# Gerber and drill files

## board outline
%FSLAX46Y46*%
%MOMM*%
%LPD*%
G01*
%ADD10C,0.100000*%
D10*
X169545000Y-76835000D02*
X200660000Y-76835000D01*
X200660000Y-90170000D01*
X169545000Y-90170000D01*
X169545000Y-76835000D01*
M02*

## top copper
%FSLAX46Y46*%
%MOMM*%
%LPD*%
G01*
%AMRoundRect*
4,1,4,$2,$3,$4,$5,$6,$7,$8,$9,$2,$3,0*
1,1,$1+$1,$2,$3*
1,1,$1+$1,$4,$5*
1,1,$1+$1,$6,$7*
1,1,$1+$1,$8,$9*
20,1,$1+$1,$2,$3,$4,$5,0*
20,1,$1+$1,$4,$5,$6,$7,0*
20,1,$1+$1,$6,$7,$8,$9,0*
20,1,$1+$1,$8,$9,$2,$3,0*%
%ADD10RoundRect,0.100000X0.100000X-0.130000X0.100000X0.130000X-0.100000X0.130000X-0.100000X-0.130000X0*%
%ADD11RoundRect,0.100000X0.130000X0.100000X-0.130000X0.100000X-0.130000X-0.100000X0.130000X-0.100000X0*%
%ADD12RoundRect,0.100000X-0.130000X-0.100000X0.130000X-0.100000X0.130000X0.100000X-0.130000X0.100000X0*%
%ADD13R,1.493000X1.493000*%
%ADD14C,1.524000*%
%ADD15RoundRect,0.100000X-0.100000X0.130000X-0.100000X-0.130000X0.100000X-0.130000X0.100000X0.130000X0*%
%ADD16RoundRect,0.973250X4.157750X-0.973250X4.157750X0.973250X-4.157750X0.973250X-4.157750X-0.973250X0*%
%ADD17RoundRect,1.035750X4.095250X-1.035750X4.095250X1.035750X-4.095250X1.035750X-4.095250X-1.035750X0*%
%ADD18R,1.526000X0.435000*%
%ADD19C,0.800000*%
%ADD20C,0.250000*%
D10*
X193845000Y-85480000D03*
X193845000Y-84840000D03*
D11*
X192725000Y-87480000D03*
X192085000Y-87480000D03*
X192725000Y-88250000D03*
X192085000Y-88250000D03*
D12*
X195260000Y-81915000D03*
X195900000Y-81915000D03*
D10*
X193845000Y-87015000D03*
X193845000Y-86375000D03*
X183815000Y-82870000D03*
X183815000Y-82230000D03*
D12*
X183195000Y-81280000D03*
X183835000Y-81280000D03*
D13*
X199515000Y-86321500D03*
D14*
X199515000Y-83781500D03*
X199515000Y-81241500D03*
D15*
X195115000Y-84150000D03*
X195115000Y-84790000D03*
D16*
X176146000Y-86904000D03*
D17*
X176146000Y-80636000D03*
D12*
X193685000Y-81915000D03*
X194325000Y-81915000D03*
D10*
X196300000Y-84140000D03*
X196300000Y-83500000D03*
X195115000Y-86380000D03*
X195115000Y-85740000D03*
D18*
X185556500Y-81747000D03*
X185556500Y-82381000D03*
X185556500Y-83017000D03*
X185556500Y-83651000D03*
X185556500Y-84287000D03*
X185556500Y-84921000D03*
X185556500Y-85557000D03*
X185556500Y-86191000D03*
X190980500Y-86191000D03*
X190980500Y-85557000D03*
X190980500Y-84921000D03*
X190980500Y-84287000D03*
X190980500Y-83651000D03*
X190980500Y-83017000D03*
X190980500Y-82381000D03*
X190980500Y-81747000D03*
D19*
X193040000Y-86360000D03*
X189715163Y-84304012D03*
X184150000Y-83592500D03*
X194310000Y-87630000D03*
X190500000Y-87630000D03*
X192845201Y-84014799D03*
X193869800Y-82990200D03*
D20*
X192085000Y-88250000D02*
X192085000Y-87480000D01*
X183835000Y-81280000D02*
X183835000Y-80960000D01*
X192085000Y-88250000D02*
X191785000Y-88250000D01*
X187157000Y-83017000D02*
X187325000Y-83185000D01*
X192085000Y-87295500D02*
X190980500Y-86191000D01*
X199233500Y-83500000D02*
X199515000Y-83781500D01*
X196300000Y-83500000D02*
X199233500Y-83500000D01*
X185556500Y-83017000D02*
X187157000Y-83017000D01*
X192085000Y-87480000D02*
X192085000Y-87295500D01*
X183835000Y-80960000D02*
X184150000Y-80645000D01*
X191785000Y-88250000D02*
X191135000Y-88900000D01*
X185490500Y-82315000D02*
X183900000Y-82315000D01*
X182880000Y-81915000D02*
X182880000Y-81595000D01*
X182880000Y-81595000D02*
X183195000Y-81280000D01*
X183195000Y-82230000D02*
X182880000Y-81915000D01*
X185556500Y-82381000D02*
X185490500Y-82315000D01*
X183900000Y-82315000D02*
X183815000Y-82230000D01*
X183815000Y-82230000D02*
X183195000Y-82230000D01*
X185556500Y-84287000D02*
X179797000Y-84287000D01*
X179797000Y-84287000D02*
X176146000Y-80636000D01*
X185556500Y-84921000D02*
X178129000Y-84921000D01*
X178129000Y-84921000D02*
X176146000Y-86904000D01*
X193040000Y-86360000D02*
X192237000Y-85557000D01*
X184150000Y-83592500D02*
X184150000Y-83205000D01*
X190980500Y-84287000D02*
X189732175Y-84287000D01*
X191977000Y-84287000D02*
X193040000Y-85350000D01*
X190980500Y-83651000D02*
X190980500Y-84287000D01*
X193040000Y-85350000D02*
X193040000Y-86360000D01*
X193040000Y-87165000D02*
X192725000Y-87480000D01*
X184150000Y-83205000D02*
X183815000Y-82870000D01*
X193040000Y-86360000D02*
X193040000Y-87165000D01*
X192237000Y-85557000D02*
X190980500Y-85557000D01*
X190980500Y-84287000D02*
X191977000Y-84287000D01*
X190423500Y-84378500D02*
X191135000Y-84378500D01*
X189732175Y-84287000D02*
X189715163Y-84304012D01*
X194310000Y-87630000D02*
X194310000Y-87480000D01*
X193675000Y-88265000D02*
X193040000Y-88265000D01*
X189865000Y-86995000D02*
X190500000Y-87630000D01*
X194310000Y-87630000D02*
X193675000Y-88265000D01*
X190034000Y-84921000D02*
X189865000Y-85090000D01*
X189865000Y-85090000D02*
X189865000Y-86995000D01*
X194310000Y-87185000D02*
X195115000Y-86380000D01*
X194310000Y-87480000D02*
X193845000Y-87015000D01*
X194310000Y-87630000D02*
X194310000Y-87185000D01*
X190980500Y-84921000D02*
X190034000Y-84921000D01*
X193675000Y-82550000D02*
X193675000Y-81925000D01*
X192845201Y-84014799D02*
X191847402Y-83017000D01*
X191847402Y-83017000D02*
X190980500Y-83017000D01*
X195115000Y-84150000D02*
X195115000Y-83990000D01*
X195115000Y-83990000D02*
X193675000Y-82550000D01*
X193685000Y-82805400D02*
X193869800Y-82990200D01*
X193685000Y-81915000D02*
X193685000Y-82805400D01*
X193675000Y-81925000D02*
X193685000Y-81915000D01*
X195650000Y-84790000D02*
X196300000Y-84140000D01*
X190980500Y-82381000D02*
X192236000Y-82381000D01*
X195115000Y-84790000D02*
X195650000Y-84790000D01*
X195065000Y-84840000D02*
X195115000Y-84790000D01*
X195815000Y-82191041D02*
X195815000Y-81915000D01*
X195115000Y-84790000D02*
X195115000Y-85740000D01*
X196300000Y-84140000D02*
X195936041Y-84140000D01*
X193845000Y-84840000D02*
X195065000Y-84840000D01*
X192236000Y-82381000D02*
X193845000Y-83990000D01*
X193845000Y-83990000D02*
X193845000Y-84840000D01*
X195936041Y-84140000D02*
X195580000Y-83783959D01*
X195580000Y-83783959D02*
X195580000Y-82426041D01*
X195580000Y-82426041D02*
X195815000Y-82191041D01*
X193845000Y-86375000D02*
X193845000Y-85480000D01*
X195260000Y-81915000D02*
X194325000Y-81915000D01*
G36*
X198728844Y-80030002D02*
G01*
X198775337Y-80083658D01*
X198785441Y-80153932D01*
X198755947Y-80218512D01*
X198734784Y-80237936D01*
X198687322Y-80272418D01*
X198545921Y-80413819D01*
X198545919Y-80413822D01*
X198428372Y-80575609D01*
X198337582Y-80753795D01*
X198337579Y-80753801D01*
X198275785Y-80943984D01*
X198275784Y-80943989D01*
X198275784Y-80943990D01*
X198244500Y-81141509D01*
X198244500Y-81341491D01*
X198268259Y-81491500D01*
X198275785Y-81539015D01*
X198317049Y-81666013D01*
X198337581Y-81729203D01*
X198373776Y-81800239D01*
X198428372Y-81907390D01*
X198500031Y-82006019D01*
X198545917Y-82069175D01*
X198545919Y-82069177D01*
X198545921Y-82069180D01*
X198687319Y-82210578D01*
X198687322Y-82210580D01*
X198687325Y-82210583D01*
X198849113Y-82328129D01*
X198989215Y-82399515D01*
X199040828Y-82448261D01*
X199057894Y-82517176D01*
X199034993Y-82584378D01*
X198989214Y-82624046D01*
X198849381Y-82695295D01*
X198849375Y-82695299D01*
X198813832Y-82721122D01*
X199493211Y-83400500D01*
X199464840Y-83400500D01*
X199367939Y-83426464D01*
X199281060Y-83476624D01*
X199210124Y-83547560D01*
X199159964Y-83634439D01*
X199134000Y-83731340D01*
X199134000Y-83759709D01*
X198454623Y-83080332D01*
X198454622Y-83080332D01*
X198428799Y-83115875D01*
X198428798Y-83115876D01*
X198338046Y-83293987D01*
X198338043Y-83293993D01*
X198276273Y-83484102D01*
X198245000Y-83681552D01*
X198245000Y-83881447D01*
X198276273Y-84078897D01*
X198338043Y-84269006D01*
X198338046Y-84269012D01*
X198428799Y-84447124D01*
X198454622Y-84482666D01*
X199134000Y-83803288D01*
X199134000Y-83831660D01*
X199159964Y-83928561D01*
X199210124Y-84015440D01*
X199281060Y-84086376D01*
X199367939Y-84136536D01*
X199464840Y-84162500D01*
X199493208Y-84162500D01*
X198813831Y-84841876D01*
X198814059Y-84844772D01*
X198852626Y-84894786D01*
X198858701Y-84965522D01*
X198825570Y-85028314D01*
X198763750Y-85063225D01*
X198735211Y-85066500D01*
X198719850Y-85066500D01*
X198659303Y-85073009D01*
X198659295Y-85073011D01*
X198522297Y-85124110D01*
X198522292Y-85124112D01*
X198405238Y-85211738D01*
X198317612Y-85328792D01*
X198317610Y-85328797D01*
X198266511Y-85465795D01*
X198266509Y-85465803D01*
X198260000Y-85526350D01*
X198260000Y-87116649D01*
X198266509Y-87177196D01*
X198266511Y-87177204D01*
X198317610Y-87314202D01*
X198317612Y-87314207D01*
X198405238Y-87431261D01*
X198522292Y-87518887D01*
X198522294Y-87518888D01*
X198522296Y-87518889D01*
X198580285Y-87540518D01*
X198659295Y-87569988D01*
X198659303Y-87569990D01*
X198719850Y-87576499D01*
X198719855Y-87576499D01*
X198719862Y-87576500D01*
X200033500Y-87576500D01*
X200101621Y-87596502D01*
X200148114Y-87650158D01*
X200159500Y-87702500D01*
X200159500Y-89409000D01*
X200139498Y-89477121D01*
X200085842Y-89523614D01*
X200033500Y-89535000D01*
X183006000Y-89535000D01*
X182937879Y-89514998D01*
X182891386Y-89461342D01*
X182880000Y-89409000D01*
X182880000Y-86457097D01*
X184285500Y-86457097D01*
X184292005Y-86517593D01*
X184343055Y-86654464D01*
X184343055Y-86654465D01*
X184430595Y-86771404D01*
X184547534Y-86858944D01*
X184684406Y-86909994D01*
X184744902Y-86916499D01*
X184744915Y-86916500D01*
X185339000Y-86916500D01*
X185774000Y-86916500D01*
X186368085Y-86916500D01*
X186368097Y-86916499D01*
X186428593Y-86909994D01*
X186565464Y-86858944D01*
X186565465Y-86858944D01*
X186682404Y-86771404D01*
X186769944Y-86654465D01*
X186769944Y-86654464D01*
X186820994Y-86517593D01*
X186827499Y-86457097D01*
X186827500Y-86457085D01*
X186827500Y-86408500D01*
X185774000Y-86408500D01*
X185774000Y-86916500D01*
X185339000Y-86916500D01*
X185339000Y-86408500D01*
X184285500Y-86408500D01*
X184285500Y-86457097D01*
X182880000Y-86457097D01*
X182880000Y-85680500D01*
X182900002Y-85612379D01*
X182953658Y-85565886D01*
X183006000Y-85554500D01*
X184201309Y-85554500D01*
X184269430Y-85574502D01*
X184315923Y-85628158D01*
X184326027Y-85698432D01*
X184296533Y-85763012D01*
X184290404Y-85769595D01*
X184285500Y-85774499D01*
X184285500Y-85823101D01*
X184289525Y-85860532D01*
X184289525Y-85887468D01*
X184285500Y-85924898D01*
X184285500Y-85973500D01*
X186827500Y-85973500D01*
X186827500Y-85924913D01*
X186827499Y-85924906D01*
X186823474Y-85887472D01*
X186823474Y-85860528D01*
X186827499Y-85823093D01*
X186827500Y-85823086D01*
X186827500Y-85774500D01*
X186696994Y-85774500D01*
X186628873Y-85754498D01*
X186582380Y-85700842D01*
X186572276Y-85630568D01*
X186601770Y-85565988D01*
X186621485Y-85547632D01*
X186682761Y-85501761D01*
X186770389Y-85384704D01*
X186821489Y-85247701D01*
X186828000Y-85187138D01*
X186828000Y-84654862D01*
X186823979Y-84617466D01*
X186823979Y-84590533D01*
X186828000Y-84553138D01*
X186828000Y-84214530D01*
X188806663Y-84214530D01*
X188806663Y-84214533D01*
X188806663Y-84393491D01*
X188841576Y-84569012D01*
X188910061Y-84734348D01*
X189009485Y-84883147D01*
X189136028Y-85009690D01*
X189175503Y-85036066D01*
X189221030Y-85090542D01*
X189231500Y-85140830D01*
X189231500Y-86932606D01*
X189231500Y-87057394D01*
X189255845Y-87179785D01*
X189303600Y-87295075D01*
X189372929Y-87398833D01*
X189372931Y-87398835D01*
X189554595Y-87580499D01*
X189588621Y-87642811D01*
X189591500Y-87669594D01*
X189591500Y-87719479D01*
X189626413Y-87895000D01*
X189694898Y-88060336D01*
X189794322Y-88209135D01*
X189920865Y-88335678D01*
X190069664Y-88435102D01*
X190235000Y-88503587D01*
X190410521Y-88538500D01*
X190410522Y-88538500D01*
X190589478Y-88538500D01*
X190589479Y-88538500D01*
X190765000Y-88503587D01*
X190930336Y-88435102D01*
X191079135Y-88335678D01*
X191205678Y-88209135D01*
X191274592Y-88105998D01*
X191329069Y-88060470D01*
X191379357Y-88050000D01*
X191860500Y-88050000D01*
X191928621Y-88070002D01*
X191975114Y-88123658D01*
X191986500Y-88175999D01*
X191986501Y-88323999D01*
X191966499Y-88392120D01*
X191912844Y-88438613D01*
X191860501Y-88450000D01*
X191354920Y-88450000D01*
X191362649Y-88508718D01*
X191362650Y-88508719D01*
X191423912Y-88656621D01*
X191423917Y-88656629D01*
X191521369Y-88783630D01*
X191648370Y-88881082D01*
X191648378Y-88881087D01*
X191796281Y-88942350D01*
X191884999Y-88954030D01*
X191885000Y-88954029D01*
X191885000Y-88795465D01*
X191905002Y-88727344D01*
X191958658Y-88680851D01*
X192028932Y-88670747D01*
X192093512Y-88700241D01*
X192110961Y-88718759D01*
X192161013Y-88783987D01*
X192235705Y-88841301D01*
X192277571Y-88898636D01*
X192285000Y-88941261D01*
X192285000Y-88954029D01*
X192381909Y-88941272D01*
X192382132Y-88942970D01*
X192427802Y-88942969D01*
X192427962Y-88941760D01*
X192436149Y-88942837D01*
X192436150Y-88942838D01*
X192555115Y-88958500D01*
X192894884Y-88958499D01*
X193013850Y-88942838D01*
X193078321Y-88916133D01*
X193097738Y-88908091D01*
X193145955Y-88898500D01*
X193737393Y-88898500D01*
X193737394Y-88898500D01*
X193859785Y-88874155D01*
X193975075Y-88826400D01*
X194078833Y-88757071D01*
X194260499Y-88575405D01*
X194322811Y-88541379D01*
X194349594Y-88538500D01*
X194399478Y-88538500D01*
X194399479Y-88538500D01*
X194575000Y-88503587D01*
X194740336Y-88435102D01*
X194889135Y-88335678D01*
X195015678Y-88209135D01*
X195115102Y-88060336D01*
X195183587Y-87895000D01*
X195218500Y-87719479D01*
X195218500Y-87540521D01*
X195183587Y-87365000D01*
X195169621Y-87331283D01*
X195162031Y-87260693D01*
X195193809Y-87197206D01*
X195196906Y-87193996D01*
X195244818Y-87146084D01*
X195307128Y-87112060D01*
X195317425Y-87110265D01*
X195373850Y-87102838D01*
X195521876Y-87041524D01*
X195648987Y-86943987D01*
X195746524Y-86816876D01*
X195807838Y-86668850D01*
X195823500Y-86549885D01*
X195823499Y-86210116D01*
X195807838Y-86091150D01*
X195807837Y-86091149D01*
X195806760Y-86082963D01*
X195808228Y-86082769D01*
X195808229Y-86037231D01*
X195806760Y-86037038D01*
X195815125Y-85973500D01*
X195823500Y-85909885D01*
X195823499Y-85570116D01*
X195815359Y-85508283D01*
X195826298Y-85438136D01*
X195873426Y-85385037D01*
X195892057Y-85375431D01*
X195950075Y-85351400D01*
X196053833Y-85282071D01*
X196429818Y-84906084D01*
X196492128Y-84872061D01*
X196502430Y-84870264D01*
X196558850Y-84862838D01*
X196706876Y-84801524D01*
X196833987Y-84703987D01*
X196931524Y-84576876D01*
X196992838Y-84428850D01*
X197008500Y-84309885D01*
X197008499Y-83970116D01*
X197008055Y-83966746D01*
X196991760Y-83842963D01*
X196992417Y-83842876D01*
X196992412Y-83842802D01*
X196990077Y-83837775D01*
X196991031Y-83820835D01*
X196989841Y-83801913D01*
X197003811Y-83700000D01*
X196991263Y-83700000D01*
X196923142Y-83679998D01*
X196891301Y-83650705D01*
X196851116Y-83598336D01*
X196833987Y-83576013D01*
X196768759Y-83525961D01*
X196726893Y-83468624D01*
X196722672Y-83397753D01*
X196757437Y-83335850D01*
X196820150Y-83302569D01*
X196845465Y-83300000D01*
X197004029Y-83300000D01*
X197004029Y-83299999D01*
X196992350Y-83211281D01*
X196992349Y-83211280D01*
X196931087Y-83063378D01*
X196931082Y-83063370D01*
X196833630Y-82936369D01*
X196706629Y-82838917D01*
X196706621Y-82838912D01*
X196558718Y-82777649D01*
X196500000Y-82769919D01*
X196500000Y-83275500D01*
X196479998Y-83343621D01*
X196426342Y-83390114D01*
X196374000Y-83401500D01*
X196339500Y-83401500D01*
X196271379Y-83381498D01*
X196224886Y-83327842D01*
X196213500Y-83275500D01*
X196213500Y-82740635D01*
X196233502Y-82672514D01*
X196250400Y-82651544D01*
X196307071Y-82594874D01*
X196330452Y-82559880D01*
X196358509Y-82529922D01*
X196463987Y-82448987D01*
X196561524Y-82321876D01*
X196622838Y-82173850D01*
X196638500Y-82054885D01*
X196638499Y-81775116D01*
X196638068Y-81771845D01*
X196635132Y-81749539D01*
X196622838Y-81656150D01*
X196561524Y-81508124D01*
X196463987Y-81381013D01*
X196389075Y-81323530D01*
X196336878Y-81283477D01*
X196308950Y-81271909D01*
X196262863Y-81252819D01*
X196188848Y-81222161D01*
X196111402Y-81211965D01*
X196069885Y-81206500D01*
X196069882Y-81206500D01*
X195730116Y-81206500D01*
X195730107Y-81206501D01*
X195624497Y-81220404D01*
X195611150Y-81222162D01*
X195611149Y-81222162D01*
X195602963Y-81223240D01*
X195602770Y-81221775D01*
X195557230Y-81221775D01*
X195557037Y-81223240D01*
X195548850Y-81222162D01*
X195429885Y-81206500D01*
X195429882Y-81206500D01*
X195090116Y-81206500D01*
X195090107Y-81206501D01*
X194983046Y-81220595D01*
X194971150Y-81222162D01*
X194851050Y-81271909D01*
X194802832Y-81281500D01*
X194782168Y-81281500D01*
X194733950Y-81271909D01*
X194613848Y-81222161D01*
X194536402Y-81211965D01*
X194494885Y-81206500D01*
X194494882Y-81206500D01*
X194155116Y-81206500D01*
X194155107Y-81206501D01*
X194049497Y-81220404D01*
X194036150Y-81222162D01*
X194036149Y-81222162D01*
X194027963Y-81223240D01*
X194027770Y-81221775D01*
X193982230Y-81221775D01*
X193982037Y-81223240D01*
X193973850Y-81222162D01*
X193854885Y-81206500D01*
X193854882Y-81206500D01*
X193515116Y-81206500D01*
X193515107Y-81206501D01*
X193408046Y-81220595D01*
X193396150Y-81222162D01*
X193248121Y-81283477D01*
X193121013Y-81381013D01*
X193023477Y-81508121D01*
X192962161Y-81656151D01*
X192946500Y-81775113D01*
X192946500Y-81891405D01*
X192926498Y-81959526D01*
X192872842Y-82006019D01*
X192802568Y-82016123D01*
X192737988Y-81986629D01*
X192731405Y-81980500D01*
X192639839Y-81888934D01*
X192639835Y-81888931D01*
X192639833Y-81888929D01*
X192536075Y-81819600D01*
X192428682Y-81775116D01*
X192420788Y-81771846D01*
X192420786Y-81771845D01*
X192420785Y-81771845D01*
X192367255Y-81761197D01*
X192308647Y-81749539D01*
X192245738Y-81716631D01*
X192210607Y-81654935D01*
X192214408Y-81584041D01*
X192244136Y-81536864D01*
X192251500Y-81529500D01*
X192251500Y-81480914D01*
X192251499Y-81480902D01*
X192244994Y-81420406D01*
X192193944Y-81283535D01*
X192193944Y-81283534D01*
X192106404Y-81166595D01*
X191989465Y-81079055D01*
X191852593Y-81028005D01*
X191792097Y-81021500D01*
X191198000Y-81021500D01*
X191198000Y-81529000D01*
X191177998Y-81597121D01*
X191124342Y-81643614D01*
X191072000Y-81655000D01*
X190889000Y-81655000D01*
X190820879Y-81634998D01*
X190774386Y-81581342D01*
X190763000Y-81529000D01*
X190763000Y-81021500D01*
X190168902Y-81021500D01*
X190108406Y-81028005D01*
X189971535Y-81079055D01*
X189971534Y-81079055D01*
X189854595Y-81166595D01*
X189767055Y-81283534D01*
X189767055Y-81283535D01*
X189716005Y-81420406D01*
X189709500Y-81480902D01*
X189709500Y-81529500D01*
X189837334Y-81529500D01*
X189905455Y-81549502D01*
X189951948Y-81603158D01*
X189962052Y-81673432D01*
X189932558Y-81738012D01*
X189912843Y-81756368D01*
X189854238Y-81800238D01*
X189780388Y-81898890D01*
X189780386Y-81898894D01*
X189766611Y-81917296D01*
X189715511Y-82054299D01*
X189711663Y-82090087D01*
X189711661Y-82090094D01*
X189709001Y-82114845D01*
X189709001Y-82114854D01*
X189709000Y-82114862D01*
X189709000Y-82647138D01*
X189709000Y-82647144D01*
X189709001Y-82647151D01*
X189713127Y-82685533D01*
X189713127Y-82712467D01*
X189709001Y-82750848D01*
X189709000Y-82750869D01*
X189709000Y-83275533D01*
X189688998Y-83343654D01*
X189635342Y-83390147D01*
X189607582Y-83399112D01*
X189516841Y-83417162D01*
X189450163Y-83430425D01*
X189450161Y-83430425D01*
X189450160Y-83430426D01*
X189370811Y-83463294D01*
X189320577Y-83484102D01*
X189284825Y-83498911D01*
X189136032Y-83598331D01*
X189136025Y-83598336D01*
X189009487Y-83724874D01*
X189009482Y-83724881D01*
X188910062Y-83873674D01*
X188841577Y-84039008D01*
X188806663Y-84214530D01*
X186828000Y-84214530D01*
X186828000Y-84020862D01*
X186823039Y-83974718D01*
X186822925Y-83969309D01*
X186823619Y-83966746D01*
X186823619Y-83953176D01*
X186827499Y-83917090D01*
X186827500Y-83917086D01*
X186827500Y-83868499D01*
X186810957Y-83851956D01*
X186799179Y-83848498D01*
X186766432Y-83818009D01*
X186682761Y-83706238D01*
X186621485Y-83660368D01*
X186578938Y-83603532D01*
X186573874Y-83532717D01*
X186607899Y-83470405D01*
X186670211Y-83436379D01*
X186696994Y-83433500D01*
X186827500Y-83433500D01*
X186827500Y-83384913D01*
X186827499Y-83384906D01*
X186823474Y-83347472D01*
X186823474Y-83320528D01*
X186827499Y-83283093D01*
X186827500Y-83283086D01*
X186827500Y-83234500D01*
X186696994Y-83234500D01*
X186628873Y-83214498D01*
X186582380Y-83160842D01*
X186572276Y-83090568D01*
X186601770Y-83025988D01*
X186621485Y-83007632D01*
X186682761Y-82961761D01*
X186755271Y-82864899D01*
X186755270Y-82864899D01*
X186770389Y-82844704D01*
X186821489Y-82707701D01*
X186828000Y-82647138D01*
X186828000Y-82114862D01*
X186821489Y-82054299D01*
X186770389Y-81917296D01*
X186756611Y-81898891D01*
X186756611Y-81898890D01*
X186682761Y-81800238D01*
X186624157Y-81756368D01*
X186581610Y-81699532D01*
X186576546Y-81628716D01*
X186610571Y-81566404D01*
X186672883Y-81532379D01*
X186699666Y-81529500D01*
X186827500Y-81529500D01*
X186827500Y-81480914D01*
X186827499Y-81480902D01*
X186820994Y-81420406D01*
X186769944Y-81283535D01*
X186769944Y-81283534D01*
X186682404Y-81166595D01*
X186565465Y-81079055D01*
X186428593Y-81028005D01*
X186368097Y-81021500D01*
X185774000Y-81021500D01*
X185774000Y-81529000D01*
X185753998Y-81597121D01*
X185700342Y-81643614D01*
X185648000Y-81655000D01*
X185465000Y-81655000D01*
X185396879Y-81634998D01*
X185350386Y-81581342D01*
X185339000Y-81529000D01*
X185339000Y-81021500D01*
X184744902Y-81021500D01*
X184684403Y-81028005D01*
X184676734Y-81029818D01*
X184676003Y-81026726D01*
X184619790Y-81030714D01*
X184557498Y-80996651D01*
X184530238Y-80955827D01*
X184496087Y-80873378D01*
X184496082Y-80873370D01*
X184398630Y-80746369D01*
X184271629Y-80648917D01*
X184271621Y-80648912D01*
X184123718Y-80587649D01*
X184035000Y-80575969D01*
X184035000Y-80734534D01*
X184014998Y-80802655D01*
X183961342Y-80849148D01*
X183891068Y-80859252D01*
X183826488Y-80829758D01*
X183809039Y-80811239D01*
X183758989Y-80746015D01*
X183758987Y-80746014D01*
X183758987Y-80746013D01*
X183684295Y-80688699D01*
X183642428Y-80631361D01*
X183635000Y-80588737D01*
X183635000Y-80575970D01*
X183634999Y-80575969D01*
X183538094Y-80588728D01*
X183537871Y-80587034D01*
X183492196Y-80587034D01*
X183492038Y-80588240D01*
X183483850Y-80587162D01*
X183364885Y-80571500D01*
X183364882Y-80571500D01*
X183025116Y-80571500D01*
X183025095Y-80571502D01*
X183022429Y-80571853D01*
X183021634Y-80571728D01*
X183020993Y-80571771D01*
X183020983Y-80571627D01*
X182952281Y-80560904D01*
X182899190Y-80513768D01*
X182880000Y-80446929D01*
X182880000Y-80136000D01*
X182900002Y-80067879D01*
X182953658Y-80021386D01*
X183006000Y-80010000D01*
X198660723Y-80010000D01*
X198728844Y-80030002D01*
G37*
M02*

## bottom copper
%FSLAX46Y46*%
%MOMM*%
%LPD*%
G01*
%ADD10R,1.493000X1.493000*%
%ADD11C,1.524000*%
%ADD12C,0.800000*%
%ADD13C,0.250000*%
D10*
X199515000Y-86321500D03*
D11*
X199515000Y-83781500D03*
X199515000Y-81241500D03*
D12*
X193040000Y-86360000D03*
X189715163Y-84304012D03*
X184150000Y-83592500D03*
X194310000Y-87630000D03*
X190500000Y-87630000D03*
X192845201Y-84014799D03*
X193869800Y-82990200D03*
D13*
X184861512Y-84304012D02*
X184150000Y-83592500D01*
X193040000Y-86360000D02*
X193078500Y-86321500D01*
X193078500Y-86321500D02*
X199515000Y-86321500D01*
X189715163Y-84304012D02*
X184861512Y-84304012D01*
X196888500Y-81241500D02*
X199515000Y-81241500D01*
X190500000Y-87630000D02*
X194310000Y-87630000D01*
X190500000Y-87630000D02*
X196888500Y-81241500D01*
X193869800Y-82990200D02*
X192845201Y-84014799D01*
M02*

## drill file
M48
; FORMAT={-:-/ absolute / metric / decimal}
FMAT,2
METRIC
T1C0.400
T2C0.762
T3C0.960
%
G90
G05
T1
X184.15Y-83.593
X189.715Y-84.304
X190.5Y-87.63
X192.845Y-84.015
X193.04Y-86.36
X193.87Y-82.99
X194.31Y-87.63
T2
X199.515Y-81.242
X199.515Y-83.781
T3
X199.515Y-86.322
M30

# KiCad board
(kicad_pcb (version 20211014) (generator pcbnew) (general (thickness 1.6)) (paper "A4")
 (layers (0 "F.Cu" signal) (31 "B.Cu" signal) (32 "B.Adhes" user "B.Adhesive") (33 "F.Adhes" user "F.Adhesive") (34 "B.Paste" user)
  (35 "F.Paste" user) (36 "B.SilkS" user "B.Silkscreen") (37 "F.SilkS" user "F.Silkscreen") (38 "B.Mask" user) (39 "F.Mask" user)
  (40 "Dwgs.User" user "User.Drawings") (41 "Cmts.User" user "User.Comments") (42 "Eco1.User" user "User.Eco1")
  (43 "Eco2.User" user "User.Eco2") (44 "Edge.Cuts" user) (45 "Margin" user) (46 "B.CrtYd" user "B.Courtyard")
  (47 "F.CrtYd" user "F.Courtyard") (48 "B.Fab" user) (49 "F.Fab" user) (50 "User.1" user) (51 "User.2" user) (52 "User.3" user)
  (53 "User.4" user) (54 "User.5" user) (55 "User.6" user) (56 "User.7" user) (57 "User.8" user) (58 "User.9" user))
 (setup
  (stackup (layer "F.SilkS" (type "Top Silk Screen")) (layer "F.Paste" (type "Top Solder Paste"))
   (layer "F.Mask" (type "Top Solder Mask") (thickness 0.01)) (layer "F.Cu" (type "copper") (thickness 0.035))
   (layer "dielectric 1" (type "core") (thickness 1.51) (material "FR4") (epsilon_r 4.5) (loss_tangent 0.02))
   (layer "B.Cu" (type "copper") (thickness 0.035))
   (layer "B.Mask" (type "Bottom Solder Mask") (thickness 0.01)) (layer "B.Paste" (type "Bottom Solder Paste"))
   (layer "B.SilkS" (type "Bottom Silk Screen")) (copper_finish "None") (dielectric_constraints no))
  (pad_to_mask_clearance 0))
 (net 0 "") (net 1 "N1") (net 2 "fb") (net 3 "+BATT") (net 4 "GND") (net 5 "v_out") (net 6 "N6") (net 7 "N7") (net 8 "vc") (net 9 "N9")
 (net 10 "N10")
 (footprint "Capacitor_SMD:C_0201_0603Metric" (layer "F.Cu") (at 193.845 85.16 90)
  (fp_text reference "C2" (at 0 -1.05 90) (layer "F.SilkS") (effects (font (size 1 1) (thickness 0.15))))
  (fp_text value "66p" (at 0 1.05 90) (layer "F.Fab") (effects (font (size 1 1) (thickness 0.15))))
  (pad "" smd roundrect (at 0.345 0 90) (size 0.318 0.36) (layers "F.Paste") (roundrect_rratio 0.25))
  (pad "" smd roundrect (at -0.345 0 90) (size 0.318 0.36) (layers "F.Paste") (roundrect_rratio 0.25))
  (pad "1" smd roundrect (at -0.32 0 90) (size 0.46 0.4) (layers "F.Cu" "F.Mask") (roundrect_rratio 0.25) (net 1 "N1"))
  (pad "2" smd roundrect (at 0.32 0 90) (size 0.46 0.4) (layers "F.Cu" "F.Mask") (roundrect_rratio 0.25) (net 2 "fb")))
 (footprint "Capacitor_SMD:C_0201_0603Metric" (layer "F.Cu") (at 192.405 87.48 180)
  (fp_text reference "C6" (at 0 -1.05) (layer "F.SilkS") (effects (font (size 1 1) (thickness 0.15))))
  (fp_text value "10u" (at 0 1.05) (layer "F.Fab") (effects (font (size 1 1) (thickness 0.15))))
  (pad "" smd roundrect (at -0.345 0 180) (size 0.318 0.36) (layers "F.Paste") (roundrect_rratio 0.25))
  (pad "" smd roundrect (at 0.345 0 180) (size 0.318 0.36) (layers "F.Paste") (roundrect_rratio 0.25))
  (pad "1" smd roundrect (at -0.32 0 180) (size 0.46 0.4) (layers "F.Cu" "F.Mask") (roundrect_rratio 0.25) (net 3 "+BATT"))
  (pad "2" smd roundrect (at 0.32 0 180) (size 0.46 0.4) (layers "F.Cu" "F.Mask") (roundrect_rratio 0.25) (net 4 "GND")))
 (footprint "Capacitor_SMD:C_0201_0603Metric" (layer "F.Cu") (at 192.405 88.25 180)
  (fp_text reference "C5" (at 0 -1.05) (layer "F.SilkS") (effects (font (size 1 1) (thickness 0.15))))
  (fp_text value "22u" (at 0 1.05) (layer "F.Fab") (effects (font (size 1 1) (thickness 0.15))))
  (pad "" smd roundrect (at 0.345 0 180) (size 0.318 0.36) (layers "F.Paste") (roundrect_rratio 0.25))
  (pad "" smd roundrect (at -0.345 0 180) (size 0.318 0.36) (layers "F.Paste") (roundrect_rratio 0.25))
  (pad "1" smd roundrect (at -0.32 0 180) (size 0.46 0.4) (layers "F.Cu" "F.Mask") (roundrect_rratio 0.25) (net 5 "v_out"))
  (pad "2" smd roundrect (at 0.32 0 180) (size 0.46 0.4) (layers "F.Cu" "F.Mask") (roundrect_rratio 0.25) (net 4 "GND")))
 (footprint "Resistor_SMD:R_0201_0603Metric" (layer "F.Cu") (at 195.58 81.915)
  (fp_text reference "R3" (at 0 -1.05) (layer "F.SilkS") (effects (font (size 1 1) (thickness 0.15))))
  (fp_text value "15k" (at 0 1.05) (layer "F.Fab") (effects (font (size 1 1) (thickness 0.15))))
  (pad "" smd roundrect (at -0.345 0) (size 0.318 0.36) (layers "F.Paste") (roundrect_rratio 0.25))
  (pad "" smd roundrect (at 0.345 0) (size 0.318 0.36) (layers "F.Paste") (roundrect_rratio 0.25))
  (pad "1" smd roundrect (at -0.32 0) (size 0.46 0.4) (layers "F.Cu" "F.Mask") (roundrect_rratio 0.25) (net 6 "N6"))
  (pad "2" smd roundrect (at 0.32 0) (size 0.46 0.4) (layers "F.Cu" "F.Mask") (roundrect_rratio 0.25) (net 2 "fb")))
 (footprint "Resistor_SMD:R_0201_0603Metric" (layer "F.Cu") (at 193.845 86.695 90)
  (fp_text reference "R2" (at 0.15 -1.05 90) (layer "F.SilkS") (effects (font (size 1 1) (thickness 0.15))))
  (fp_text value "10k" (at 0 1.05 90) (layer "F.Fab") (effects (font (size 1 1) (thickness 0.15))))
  (pad "" smd roundrect (at -0.345 0 90) (size 0.318 0.36) (layers "F.Paste") (roundrect_rratio 0.25))
  (pad "" smd roundrect (at 0.345 0 90) (size 0.318 0.36) (layers "F.Paste") (roundrect_rratio 0.25))
  (pad "1" smd roundrect (at -0.32 0 90) (size 0.46 0.4) (layers "F.Cu" "F.Mask") (roundrect_rratio 0.25) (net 5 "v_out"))
  (pad "2" smd roundrect (at 0.32 0 90) (size 0.46 0.4) (layers "F.Cu" "F.Mask") (roundrect_rratio 0.25) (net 1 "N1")))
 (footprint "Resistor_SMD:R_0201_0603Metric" (layer "F.Cu") (at 183.815 82.55 90)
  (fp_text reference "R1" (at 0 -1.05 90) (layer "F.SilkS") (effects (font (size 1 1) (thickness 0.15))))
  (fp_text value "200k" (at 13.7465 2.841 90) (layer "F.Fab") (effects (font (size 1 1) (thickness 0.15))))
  (pad "" smd roundrect (at -0.345 0 90) (size 0.318 0.36) (layers "F.Paste") (roundrect_rratio 0.25))
  (pad "" smd roundrect (at 0.345 0 90) (size 0.318 0.36) (layers "F.Paste") (roundrect_rratio 0.25))
  (pad "1" smd roundrect (at -0.32 0 90) (size 0.46 0.4) (layers "F.Cu" "F.Mask") (roundrect_rratio 0.25) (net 3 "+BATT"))
  (pad "2" smd roundrect (at 0.32 0 90) (size 0.46 0.4) (layers "F.Cu" "F.Mask") (roundrect_rratio 0.25) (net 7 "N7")))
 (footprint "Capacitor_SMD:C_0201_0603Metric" (layer "F.Cu") (at 183.515 81.28)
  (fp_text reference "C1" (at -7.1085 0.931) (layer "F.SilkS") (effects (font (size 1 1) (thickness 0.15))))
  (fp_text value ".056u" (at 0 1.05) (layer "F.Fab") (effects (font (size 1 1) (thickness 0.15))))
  (pad "" smd roundrect (at 0.345 0) (size 0.318 0.36) (layers "F.Paste") (roundrect_rratio 0.25))
  (pad "" smd roundrect (at -0.345 0) (size 0.318 0.36) (layers "F.Paste") (roundrect_rratio 0.25))
  (pad "1" smd roundrect (at -0.32 0) (size 0.46 0.4) (layers "F.Cu" "F.Mask") (roundrect_rratio 0.25) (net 7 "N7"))
  (pad "2" smd roundrect (at 0.32 0) (size 0.46 0.4) (layers "F.Cu" "F.Mask") (roundrect_rratio 0.25) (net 4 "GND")))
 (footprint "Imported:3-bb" (layer "F.Cu") (at 199.515 86.3215 90)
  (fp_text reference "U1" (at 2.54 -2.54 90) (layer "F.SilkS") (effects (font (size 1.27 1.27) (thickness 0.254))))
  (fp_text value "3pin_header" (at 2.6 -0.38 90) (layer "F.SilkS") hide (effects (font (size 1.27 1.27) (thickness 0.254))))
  (pad "1" thru_hole rect (at 0 0 90) (size 1.493 1.493) (drill 0.96) (layers *.Cu *.Mask) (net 3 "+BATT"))
  (pad "2" thru_hole circle (at 2.54 0 90) (size 1.524 1.524) (drill 0.762) (layers *.Cu *.Mask) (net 4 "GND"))
  (pad "3" thru_hole circle (at 5.08 0 90) (size 1.524 1.524) (drill 0.762) (layers *.Cu *.Mask) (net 5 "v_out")))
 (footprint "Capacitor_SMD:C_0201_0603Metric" (layer "F.Cu") (at 195.115 84.47 -90)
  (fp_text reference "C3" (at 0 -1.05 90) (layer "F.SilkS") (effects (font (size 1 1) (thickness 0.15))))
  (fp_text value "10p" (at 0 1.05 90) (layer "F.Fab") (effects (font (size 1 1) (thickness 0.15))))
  (pad "" smd roundrect (at -0.345 0 270) (size 0.318 0.36) (layers "F.Paste") (roundrect_rratio 0.25))
  (pad "" smd roundrect (at 0.345 0 270) (size 0.318 0.36) (layers "F.Paste") (roundrect_rratio 0.25))
  (pad "1" smd roundrect (at -0.32 0 270) (size 0.46 0.4) (layers "F.Cu" "F.Mask") (roundrect_rratio 0.25) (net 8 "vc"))
  (pad "2" smd roundrect (at 0.32 0 270) (size 0.46 0.4) (layers "F.Cu" "F.Mask") (roundrect_rratio 0.25) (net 2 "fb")))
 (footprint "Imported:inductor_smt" (layer "F.Cu") (at 183.515 91.2075 90)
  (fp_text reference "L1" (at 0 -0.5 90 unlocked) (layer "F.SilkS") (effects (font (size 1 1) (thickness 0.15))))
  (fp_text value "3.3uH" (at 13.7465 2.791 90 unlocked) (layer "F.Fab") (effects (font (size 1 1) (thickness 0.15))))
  (pad "1" smd roundrect (at 4.3035 -7.369 90) (size 3.893 10.262) (layers "F.Cu" "F.Paste" "F.Mask") (roundrect_rratio 0.25) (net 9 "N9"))
  (pad "2" smd roundrect (at 10.5715 -7.369 90) (size 4.143 10.262) (layers "F.Cu" "F.Paste" "F.Mask") (roundrect_rratio 0.25)
   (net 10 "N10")))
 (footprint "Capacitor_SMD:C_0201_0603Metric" (layer "F.Cu") (at 194.005 81.915)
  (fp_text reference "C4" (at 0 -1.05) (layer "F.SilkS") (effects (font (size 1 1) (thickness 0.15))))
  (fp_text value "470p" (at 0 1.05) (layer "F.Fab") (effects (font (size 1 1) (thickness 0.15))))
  (pad "" smd roundrect (at -0.345 0) (size 0.318 0.36) (layers "F.Paste") (roundrect_rratio 0.25))
  (pad "" smd roundrect (at 0.345 0) (size 0.318 0.36) (layers "F.Paste") (roundrect_rratio 0.25))
  (pad "1" smd roundrect (at -0.32 0) (size 0.46 0.4) (layers "F.Cu" "F.Mask") (roundrect_rratio 0.25) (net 8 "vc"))
  (pad "2" smd roundrect (at 0.32 0) (size 0.46 0.4) (layers "F.Cu" "F.Mask") (roundrect_rratio 0.25) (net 6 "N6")))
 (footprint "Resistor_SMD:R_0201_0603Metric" (layer "F.Cu") (at 196.3 83.82 90)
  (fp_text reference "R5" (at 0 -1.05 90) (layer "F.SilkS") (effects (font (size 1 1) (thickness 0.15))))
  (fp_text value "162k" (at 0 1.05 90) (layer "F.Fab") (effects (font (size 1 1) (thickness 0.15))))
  (pad "" smd roundrect (at 0.345 0 90) (size 0.318 0.36) (layers "F.Paste") (roundrect_rratio 0.25))
  (pad "" smd roundrect (at -0.345 0 90) (size 0.318 0.36) (layers "F.Paste") (roundrect_rratio 0.25))
  (pad "1" smd roundrect (at -0.32 0 90) (size 0.46 0.4) (layers "F.Cu" "F.Mask") (roundrect_rratio 0.25) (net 2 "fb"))
  (pad "2" smd roundrect (at 0.32 0 90) (size 0.46 0.4) (layers "F.Cu" "F.Mask") (roundrect_rratio 0.25) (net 4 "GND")))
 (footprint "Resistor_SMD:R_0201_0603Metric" (layer "F.Cu") (at 195.115 86.06 90)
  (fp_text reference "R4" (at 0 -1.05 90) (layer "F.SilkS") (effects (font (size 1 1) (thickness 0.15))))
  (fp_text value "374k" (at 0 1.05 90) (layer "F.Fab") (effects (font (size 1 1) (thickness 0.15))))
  (pad "" smd roundrect (at 0.345 0 90) (size 0.318 0.36) (layers "F.Paste") (roundrect_rratio 0.25))
  (pad "" smd roundrect (at -0.345 0 90) (size 0.318 0.36) (layers "F.Paste") (roundrect_rratio 0.25))
  (pad "1" smd roundrect (at -0.32 0 90) (size 0.46 0.4) (layers "F.Cu" "F.Mask") (roundrect_rratio 0.25) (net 5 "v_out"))
  (pad "2" smd roundrect (at 0.32 0 90) (size 0.46 0.4) (layers "F.Cu" "F.Mask") (roundrect_rratio 0.25) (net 2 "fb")))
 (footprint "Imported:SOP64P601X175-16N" (layer "F.Cu") (at 188.2685 83.969)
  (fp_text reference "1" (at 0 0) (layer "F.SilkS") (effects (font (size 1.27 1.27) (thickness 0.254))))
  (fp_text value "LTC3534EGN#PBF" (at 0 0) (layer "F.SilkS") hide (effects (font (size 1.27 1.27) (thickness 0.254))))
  (pad "1" smd rect (at -2.712 -2.222 90) (size 0.435 1.526) (layers "F.Cu" "F.Paste" "F.Mask") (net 4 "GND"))
  (pad "2" smd rect (at -2.712 -1.588 90) (size 0.435 1.526) (layers "F.Cu" "F.Paste" "F.Mask") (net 7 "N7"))
  (pad "3" smd rect (at -2.712 -0.952 90) (size 0.435 1.526) (layers "F.Cu" "F.Paste" "F.Mask") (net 4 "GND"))
  (pad "4" smd rect (at -2.712 -0.318 90) (size 0.435 1.526) (layers "F.Cu" "F.Paste" "F.Mask") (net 4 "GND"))
  (pad "5" smd rect (at -2.712 0.318 90) (size 0.435 1.526) (layers "F.Cu" "F.Paste" "F.Mask") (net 10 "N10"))
  (pad "6" smd rect (at -2.712 0.952 90) (size 0.435 1.526) (layers "F.Cu" "F.Paste" "F.Mask") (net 9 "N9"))
  (pad "7" smd rect (at -2.712 1.588 90) (size 0.435 1.526) (layers "F.Cu" "F.Paste" "F.Mask") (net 4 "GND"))
  (pad "8" smd rect (at -2.712 2.222 90) (size 0.435 1.526) (layers "F.Cu" "F.Paste" "F.Mask") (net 4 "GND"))
  (pad "9" smd rect (at 2.712 2.222 90) (size 0.435 1.526) (layers "F.Cu" "F.Paste" "F.Mask") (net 4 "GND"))
  (pad "10" smd rect (at 2.712 1.588 90) (size 0.435 1.526) (layers "F.Cu" "F.Paste" "F.Mask") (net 3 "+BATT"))
  (pad "11" smd rect (at 2.712 0.952 90) (size 0.435 1.526) (layers "F.Cu" "F.Paste" "F.Mask") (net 5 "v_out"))
  (pad "12" smd rect (at 2.712 0.318 90) (size 0.435 1.526) (layers "F.Cu" "F.Paste" "F.Mask") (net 3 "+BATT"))
  (pad "13" smd rect (at 2.712 -0.318 90) (size 0.435 1.526) (layers "F.Cu" "F.Paste" "F.Mask") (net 3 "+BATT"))
  (pad "14" smd rect (at 2.712 -0.952 90) (size 0.435 1.526) (layers "F.Cu" "F.Paste" "F.Mask") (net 8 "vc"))
  (pad "15" smd rect (at 2.712 -1.588 90) (size 0.435 1.526) (layers "F.Cu" "F.Paste" "F.Mask") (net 2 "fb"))
  (pad "16" smd rect (at 2.712 -2.222 90) (size 0.435 1.526) (layers "F.Cu" "F.Paste" "F.Mask") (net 4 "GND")))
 (gr_rect (start 169.545 90.17) (end 200.66 76.835) (layer "Edge.Cuts") (width 0.1) (fill none))
 (segment (start 192.085 88.25) (end 192.085 87.48) (width 0.25) (layer "F.Cu") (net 4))
 (segment (start 183.835 81.28) (end 183.835 80.96) (width 0.25) (layer "F.Cu") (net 4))
 (segment (start 192.085 88.25) (end 191.785 88.25) (width 0.25) (layer "F.Cu") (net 4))
 (segment (start 187.157 83.017) (end 187.325 83.185) (width 0.25) (layer "F.Cu") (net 4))
 (segment (start 192.085 87.2955) (end 190.9805 86.191) (width 0.25) (layer "F.Cu") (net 4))
 (segment (start 199.2335 83.5) (end 199.515 83.7815) (width 0.25) (layer "F.Cu") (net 4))
 (segment (start 196.3 83.5) (end 199.2335 83.5) (width 0.25) (layer "F.Cu") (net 4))
 (segment (start 185.5565 83.017) (end 187.157 83.017) (width 0.25) (layer "F.Cu") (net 4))
 (segment (start 192.085 87.48) (end 192.085 87.2955) (width 0.25) (layer "F.Cu") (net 4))
 (segment (start 183.835 80.96) (end 184.15 80.645) (width 0.25) (layer "F.Cu") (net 4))
 (segment (start 191.785 88.25) (end 191.135 88.9) (width 0.25) (layer "F.Cu") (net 4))
 (segment (start 185.4905 82.315) (end 183.9 82.315) (width 0.25) (layer "F.Cu") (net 7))
 (segment (start 182.88 81.915) (end 182.88 81.595) (width 0.25) (layer "F.Cu") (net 7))
 (segment (start 182.88 81.595) (end 183.195 81.28) (width 0.25) (layer "F.Cu") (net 7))
 (segment (start 183.195 82.23) (end 182.88 81.915) (width 0.25) (layer "F.Cu") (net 7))
 (segment (start 185.5565 82.381) (end 185.4905 82.315) (width 0.25) (layer "F.Cu") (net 7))
 (segment (start 183.9 82.315) (end 183.815 82.23) (width 0.25) (layer "F.Cu") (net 7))
 (segment (start 183.815 82.23) (end 183.195 82.23) (width 0.25) (layer "F.Cu") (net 7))
 (segment (start 185.5565 84.287) (end 179.797 84.287) (width 0.25) (layer "F.Cu") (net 10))
 (segment (start 179.797 84.287) (end 176.146 80.636) (width 0.25) (layer "F.Cu") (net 10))
 (segment (start 185.5565 84.921) (end 178.129 84.921) (width 0.25) (layer "F.Cu") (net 9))
 (segment (start 178.129 84.921) (end 176.146 86.904) (width 0.25) (layer "F.Cu") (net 9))
 (segment (start 193.04 86.36) (end 192.237 85.557) (width 0.25) (layer "F.Cu") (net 3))
 (segment (start 184.15 83.5925) (end 184.15 83.205) (width 0.25) (layer "F.Cu") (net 3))
 (segment (start 190.9805 84.287) (end 189.732175 84.287) (width 0.25) (layer "F.Cu") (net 3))
 (segment (start 191.977 84.287) (end 193.04 85.35) (width 0.25) (layer "F.Cu") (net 3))
 (segment (start 190.9805 83.651) (end 190.9805 84.287) (width 0.25) (layer "F.Cu") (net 3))
 (segment (start 193.04 85.35) (end 193.04 86.36) (width 0.25) (layer "F.Cu") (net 3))
 (segment (start 193.04 87.165) (end 192.725 87.48) (width 0.25) (layer "F.Cu") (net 3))
 (segment (start 184.15 83.205) (end 183.815 82.87) (width 0.25) (layer "F.Cu") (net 3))
 (segment (start 193.04 86.36) (end 193.04 87.165) (width 0.25) (layer "F.Cu") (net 3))
 (segment (start 192.237 85.557) (end 190.9805 85.557) (width 0.25) (layer "F.Cu") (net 3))
 (segment (start 190.9805 84.287) (end 191.977 84.287) (width 0.25) (layer "F.Cu") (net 3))
 (segment (start 190.4235 84.3785) (end 191.135 84.3785) (width 0.25) (layer "F.Cu") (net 3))
 (segment (start 189.732175 84.287) (end 189.715163 84.304012) (width 0.25) (layer "F.Cu") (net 3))
 (via (at 193.04 86.36) (size 0.8) (drill 0.4) (layers "F.Cu" "B.Cu") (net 3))
 (via (at 189.715163 84.304012) (size 0.8) (drill 0.4) (layers "F.Cu" "B.Cu") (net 3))
 (via (at 184.15 83.5925) (size 0.8) (drill 0.4) (layers "F.Cu" "B.Cu") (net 3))
 (segment (start 184.861512 84.304012) (end 184.15 83.5925) (width 0.25) (layer "B.Cu") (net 3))
 (segment (start 193.04 86.36) (end 193.0785 86.3215) (width 0.25) (layer "B.Cu") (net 3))
 (segment (start 193.0785 86.3215) (end 199.515 86.3215) (width 0.25) (layer "B.Cu") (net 3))
 (segment (start 189.715163 84.304012) (end 184.861512 84.304012) (width 0.25) (layer "B.Cu") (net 3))
 (segment (start 194.31 87.63) (end 194.31 87.48) (width 0.25) (layer "F.Cu") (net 5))
 (segment (start 193.675 88.265) (end 193.04 88.265) (width 0.25) (layer "F.Cu") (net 5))
 (segment (start 189.865 86.995) (end 190.5 87.63) (width 0.25) (layer "F.Cu") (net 5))
 (segment (start 194.31 87.63) (end 193.675 88.265) (width 0.25) (layer "F.Cu") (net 5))
 (segment (start 190.034 84.921) (end 189.865 85.09) (width 0.25) (layer "F.Cu") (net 5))
 (segment (start 189.865 85.09) (end 189.865 86.995) (width 0.25) (layer "F.Cu") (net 5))
 (segment (start 194.31 87.185) (end 195.115 86.38) (width 0.25) (layer "F.Cu") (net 5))
 (segment (start 194.31 87.48) (end 193.845 87.015) (width 0.25) (layer "F.Cu") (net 5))
 (segment (start 194.31 87.63) (end 194.31 87.185) (width 0.25) (layer "F.Cu") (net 5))
 (segment (start 190.9805 84.921) (end 190.034 84.921) (width 0.25) (layer "F.Cu") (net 5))
 (via (at 194.31 87.63) (size 0.8) (drill 0.4) (layers "F.Cu" "B.Cu") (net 5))
 (via (at 190.5 87.63) (size 0.8) (drill 0.4) (layers "F.Cu" "B.Cu") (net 5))
 (segment (start 196.8885 81.2415) (end 199.515 81.2415) (width 0.25) (layer "B.Cu") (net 5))
 (segment (start 190.5 87.63) (end 194.31 87.63) (width 0.25) (layer "B.Cu") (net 5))
 (segment (start 190.5 87.63) (end 196.8885 81.2415) (width 0.25) (layer "B.Cu") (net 5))
 (segment (start 193.675 82.55) (end 193.675 81.925) (width 0.25) (layer "F.Cu") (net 8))
 (segment (start 192.845201 84.014799) (end 191.847402 83.017) (width 0.25) (layer "F.Cu") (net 8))
 (segment (start 191.847402 83.017) (end 190.9805 83.017) (width 0.25) (layer "F.Cu") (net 8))
 (segment (start 195.115 84.15) (end 195.115 83.99) (width 0.25) (layer "F.Cu") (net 8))
 (segment (start 195.115 83.99) (end 193.675 82.55) (width 0.25) (layer "F.Cu") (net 8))
 (segment (start 193.685 82.8054) (end 193.8698 82.9902) (width 0.25) (layer "F.Cu") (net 8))
 (segment (start 193.685 81.915) (end 193.685 82.8054) (width 0.25) (layer "F.Cu") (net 8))
 (segment (start 193.675 81.925) (end 193.685 81.915) (width 0.25) (layer "F.Cu") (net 8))
 (via (at 192.845201 84.014799) (size 0.8) (drill 0.4) (layers "F.Cu" "B.Cu") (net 8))
 (via (at 193.8698 82.9902) (size 0.8) (drill 0.4) (layers "F.Cu" "B.Cu") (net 8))
 (segment (start 193.8698 82.9902) (end 192.845201 84.014799) (width 0.25) (layer "B.Cu") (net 8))
 (segment (start 195.65 84.79) (end 196.3 84.14) (width 0.25) (layer "F.Cu") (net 2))
 (segment (start 190.9805 82.381) (end 192.236 82.381) (width 0.25) (layer "F.Cu") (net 2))
 (segment (start 195.115 84.79) (end 195.65 84.79) (width 0.25) (layer "F.Cu") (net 2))
 (segment (start 195.065 84.84) (end 195.115 84.79) (width 0.25) (layer "F.Cu") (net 2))
 (segment (start 195.815 82.191041) (end 195.815 81.915) (width 0.25) (layer "F.Cu") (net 2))
 (segment (start 195.115 84.79) (end 195.115 85.74) (width 0.25) (layer "F.Cu") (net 2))
 (segment (start 196.3 84.14) (end 195.936041 84.14) (width 0.25) (layer "F.Cu") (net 2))
 (segment (start 193.845 84.84) (end 195.065 84.84) (width 0.25) (layer "F.Cu") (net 2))
 (segment (start 192.236 82.381) (end 193.845 83.99) (width 0.25) (layer "F.Cu") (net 2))
 (segment (start 193.845 83.99) (end 193.845 84.84) (width 0.25) (layer "F.Cu") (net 2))
 (segment (start 195.936041 84.14) (end 195.58 83.783959) (width 0.25) (layer "F.Cu") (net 2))
 (segment (start 195.58 83.783959) (end 195.58 82.426041) (width 0.25) (layer "F.Cu") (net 2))
 (segment (start 195.58 82.426041) (end 195.815 82.191041) (width 0.25) (layer "F.Cu") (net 2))
 (segment (start 193.845 86.375) (end 193.845 85.48) (width 0.25) (layer "F.Cu") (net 1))
 (segment (start 195.26 81.915) (end 194.325 81.915) (width 0.25) (layer "F.Cu") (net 6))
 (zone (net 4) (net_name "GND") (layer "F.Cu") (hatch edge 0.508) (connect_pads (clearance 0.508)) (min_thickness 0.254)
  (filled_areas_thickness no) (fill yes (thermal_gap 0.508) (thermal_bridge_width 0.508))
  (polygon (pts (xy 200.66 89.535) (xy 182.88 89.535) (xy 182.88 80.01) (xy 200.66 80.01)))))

